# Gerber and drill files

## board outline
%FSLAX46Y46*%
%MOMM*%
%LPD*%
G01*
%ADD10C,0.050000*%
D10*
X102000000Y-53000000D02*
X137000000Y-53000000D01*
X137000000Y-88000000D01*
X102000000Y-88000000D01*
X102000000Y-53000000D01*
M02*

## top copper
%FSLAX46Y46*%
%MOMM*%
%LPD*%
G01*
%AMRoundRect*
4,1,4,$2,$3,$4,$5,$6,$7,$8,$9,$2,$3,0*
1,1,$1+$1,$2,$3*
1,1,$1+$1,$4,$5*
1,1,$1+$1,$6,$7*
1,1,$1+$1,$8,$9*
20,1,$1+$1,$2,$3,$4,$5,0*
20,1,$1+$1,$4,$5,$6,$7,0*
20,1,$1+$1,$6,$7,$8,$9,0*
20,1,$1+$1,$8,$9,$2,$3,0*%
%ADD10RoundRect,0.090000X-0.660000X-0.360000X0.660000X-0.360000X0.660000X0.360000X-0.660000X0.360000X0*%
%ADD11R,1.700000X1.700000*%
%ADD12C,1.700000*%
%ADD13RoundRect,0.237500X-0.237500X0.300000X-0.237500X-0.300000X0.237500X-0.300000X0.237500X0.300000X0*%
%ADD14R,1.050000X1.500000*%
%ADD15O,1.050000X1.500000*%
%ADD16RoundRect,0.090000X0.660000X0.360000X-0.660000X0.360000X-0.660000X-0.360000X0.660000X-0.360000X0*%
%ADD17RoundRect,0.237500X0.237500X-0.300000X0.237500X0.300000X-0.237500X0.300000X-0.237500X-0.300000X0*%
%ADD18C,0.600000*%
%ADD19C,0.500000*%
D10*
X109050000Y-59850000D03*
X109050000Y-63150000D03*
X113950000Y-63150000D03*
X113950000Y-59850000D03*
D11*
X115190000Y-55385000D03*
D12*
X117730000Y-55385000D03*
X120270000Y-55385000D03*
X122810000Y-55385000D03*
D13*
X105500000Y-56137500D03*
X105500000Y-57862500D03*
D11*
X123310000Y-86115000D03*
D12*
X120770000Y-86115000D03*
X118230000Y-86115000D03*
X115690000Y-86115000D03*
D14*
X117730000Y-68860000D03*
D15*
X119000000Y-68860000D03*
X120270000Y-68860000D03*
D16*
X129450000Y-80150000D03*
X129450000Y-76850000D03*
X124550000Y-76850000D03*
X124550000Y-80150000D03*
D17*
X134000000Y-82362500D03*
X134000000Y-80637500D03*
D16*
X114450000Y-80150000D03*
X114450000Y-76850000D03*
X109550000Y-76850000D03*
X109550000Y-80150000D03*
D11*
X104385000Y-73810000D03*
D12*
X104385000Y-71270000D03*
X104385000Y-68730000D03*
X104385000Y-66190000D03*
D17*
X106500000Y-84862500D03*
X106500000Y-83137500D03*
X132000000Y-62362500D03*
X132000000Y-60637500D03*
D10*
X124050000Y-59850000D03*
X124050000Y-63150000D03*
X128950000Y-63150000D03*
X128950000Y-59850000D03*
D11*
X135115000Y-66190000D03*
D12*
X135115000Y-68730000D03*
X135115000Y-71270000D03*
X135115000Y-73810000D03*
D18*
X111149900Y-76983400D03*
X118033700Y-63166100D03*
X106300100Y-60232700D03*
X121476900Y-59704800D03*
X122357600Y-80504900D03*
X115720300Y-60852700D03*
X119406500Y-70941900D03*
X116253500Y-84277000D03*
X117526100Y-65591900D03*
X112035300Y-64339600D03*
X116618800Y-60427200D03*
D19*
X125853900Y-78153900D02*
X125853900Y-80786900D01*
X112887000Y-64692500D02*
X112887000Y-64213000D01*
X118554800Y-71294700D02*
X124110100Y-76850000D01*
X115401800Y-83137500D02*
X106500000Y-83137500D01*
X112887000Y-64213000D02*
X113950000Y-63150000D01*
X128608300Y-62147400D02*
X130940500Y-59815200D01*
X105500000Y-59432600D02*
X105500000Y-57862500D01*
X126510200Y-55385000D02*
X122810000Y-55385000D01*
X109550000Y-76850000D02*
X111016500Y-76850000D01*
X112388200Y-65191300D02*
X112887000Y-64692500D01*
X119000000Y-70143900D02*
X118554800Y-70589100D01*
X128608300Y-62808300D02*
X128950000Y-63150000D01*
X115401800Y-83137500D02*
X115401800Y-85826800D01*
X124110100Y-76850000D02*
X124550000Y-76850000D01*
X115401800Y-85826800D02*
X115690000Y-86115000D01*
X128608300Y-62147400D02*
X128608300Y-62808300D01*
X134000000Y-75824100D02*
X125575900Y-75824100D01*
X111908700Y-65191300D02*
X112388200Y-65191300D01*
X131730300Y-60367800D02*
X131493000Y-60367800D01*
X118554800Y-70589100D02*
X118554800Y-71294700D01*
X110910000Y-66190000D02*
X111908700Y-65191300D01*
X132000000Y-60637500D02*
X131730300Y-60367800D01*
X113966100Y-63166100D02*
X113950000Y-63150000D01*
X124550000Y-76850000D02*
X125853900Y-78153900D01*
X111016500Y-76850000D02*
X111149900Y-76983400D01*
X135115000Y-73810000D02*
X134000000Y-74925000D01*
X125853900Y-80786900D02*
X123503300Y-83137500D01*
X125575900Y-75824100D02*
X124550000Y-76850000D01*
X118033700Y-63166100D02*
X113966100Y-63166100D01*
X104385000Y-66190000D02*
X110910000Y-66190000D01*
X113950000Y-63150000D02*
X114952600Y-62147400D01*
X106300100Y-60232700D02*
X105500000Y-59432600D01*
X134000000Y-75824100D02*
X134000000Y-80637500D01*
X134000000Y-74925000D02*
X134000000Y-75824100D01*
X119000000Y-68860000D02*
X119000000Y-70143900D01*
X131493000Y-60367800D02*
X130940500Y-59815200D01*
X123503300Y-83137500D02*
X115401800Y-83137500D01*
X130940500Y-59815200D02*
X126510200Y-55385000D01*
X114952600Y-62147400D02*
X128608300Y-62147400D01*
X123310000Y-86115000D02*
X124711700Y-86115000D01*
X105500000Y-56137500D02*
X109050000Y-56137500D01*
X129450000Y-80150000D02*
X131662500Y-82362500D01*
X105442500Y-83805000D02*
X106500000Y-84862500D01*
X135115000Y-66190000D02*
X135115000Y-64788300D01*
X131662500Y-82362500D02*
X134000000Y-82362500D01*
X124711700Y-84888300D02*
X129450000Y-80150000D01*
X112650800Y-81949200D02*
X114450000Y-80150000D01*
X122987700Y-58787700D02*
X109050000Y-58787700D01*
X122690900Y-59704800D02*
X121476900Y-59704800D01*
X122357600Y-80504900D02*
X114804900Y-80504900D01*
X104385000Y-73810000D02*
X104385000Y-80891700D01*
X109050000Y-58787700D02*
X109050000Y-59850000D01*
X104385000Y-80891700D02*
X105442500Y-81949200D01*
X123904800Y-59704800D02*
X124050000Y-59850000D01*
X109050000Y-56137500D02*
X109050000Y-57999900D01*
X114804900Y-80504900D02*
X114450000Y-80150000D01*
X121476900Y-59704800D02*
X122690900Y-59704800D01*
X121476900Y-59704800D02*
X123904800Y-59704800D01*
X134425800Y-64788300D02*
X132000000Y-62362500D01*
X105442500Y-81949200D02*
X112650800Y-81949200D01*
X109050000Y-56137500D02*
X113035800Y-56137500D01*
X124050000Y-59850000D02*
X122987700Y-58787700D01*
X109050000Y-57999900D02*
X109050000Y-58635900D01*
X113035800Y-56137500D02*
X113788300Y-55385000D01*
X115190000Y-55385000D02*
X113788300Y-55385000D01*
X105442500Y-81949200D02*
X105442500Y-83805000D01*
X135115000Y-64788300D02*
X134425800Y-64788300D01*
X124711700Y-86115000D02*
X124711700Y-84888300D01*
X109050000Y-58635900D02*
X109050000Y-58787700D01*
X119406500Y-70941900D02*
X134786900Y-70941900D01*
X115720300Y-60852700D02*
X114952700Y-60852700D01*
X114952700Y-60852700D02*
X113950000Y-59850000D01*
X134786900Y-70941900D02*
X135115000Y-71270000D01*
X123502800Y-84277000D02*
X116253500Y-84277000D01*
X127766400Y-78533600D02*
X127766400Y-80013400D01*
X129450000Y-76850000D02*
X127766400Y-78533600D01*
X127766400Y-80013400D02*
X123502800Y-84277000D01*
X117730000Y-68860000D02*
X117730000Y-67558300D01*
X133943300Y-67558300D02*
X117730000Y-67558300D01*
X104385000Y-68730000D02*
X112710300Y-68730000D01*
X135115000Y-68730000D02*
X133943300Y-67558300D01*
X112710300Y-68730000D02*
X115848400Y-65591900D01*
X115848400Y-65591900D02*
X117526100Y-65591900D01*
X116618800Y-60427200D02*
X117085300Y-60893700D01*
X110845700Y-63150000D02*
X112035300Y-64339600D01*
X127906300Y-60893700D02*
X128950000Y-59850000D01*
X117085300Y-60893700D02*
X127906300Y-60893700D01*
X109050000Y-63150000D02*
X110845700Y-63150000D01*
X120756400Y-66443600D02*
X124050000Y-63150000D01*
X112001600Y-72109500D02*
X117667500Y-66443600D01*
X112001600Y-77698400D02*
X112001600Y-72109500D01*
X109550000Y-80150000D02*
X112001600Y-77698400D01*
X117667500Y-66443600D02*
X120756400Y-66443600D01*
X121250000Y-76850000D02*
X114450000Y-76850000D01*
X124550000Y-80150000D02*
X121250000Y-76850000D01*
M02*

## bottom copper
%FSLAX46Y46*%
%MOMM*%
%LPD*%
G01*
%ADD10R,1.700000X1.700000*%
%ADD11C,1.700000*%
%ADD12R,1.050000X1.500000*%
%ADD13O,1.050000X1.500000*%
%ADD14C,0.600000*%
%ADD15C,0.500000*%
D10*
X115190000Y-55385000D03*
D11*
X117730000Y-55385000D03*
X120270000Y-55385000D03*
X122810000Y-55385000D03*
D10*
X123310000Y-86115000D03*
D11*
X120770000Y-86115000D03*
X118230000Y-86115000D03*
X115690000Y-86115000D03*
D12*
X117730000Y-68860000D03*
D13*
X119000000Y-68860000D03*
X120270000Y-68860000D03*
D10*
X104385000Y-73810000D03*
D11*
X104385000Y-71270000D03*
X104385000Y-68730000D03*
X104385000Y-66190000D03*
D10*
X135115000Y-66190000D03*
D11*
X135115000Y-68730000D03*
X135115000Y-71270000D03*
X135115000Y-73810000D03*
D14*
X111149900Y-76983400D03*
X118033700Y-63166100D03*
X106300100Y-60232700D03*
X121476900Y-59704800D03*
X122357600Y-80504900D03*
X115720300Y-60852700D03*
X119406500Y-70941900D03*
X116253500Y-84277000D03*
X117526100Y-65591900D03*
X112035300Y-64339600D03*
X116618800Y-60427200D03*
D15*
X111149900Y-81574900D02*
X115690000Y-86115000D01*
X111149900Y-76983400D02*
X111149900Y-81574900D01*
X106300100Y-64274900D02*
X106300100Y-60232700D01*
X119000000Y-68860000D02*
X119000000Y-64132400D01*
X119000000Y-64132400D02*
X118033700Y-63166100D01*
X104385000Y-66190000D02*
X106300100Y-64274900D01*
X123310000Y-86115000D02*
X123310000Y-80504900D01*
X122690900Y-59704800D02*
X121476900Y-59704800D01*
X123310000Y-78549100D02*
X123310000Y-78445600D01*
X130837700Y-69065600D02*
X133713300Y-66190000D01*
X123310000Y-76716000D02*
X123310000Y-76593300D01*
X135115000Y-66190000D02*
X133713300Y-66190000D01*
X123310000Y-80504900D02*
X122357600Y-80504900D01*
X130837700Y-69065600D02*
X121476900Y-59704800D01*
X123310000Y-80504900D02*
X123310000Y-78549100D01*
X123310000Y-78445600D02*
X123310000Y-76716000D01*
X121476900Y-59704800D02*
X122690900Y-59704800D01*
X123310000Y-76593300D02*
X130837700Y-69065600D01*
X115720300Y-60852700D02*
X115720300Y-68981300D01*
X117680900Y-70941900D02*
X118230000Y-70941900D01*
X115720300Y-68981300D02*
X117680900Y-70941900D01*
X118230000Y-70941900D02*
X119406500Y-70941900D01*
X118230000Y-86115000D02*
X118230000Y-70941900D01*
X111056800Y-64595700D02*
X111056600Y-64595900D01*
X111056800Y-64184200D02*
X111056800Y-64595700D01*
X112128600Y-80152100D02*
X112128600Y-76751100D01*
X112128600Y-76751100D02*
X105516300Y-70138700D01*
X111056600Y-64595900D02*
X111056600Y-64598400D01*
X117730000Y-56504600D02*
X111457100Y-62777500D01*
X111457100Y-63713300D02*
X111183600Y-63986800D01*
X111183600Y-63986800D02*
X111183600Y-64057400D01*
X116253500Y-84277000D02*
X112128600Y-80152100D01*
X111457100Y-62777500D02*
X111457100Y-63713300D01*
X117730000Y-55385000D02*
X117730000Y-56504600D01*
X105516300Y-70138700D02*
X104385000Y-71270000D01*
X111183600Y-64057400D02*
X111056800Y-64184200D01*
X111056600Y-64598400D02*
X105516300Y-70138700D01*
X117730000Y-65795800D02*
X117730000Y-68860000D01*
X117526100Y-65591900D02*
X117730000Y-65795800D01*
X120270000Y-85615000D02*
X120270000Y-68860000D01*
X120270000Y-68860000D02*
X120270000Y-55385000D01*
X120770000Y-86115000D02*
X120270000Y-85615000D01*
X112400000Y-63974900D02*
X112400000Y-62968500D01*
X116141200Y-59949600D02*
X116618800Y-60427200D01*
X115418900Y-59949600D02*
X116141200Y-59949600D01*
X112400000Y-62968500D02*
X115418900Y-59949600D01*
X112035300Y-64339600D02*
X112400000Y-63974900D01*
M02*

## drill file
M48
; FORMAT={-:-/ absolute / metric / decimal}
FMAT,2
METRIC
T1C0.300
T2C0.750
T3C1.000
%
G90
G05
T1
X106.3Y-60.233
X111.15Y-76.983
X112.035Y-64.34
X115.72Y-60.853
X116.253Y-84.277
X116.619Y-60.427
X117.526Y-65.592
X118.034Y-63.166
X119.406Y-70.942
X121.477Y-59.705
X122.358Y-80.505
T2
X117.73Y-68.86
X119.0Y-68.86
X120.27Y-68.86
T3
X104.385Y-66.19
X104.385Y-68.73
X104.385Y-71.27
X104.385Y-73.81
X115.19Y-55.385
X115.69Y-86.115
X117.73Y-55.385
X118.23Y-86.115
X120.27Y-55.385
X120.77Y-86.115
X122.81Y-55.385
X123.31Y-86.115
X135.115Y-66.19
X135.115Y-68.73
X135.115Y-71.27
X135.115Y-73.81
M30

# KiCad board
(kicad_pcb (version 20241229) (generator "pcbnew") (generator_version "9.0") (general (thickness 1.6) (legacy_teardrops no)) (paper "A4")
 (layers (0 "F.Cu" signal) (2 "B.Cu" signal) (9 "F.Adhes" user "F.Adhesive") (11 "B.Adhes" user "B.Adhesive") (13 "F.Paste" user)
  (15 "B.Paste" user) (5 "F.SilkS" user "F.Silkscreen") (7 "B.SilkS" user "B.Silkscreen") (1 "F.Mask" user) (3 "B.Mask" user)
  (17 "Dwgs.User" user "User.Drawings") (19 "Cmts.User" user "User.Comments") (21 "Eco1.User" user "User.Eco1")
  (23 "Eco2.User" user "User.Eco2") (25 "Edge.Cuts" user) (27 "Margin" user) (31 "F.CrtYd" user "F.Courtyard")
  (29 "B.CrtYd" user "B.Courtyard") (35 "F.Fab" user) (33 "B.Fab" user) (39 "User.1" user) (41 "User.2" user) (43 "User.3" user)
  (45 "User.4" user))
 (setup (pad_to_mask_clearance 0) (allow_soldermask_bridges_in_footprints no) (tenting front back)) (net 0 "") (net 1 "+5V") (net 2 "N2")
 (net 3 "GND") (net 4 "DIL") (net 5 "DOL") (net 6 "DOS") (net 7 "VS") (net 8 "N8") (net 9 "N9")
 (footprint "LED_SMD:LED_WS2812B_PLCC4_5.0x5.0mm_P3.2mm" (layer "F.Cu") (at 111.5 61.5)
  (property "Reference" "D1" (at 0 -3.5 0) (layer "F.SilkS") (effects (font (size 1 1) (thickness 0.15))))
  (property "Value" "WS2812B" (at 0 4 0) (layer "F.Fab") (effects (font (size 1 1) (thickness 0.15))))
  (pad "1" smd roundrect (at -2.45 -1.65) (size 1.5 0.9) (layers "F.Cu" "F.Mask" "F.Paste") (roundrect_rratio 0.1) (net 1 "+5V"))
  (pad "2" smd roundrect (at -2.45 1.65) (size 1.5 0.9) (layers "F.Cu" "F.Mask" "F.Paste") (roundrect_rratio 0.1) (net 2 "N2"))
  (pad "3" smd roundrect (at 2.45 1.65) (size 1.5 0.9) (layers "F.Cu" "F.Mask" "F.Paste") (roundrect_rratio 0.1) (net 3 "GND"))
  (pad "4" smd roundrect (at 2.45 -1.65) (size 1.5 0.9) (layers "F.Cu" "F.Mask" "F.Paste") (roundrect_rratio 0.1) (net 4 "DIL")))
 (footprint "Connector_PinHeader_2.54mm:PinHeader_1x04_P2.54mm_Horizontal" (layer "F.Cu") (at 115.19 55.385 90)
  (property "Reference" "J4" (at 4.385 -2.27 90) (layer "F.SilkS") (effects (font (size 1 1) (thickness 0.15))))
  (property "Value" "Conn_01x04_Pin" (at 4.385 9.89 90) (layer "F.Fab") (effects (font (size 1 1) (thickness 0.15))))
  (pad "1" thru_hole rect (at 0 0 90) (size 1.7 1.7) (drill 1) (layers "*.Cu" "*.Mask") (remove_unused_layers no) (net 1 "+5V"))
  (pad "2" thru_hole circle (at 0 2.54 90) (size 1.7 1.7) (drill 1) (layers "*.Cu" "*.Mask") (remove_unused_layers no) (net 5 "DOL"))
  (pad "3" thru_hole circle (at 0 5.08 90) (size 1.7 1.7) (drill 1) (layers "*.Cu" "*.Mask") (remove_unused_layers no) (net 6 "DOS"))
  (pad "4" thru_hole circle (at 0 7.62 90) (size 1.7 1.7) (drill 1) (layers "*.Cu" "*.Mask") (remove_unused_layers no) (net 3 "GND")))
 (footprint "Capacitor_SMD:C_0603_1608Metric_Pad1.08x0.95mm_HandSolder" (layer "F.Cu") (at 105.5 57 -90)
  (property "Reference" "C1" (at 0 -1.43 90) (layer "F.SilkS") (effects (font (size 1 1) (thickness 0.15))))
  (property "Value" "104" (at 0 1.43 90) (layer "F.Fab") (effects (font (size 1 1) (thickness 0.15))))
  (pad "1" smd roundrect (at -0.8625 0 270) (size 1.075 0.95) (layers "F.Cu" "F.Mask" "F.Paste") (roundrect_rratio 0.25) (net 1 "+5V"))
  (pad "2" smd roundrect (at 0.8625 0 270) (size 1.075 0.95) (layers "F.Cu" "F.Mask" "F.Paste") (roundrect_rratio 0.25) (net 3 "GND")))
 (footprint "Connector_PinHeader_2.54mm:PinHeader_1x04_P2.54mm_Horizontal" (layer "F.Cu") (at 123.31 86.115 -90)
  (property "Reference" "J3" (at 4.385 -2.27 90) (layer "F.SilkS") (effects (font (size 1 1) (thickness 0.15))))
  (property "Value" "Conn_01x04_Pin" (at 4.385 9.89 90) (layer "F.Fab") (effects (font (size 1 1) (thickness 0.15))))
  (pad "1" thru_hole rect (at 0 0 270) (size 1.7 1.7) (drill 1) (layers "*.Cu" "*.Mask") (remove_unused_layers no) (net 1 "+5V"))
  (pad "2" thru_hole circle (at 0 2.54 270) (size 1.7 1.7) (drill 1) (layers "*.Cu" "*.Mask") (remove_unused_layers no) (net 6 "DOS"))
  (pad "3" thru_hole circle (at 0 5.08 270) (size 1.7 1.7) (drill 1) (layers "*.Cu" "*.Mask") (remove_unused_layers no) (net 4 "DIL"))
  (pad "4" thru_hole circle (at 0 7.62 270) (size 1.7 1.7) (drill 1) (layers "*.Cu" "*.Mask") (remove_unused_layers no) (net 3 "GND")))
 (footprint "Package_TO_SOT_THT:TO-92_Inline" (layer "F.Cu") (at 117.73 68.86)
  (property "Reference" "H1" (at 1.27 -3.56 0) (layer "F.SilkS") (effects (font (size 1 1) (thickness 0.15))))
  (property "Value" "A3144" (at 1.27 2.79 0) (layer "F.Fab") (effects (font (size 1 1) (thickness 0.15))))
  (pad "1" thru_hole rect (at 0 0) (size 1.05 1.5) (drill 0.75) (layers "*.Cu" "*.Mask") (remove_unused_layers no) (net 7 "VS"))
  (pad "2" thru_hole oval (at 1.27 0) (size 1.05 1.5) (drill 0.75) (layers "*.Cu" "*.Mask") (remove_unused_layers no) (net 3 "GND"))
  (pad "3" thru_hole oval (at 2.54 0) (size 1.05 1.5) (drill 0.75) (layers "*.Cu" "*.Mask") (remove_unused_layers no) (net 6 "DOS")))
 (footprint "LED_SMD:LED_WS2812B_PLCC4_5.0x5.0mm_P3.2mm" (layer "F.Cu") (at 127 78.5 180)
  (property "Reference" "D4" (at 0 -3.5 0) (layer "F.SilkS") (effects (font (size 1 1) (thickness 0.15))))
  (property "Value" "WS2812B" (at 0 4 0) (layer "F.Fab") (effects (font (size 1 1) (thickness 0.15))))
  (pad "1" smd roundrect (at -2.45 -1.65 180) (size 1.5 0.9) (layers "F.Cu" "F.Mask" "F.Paste") (roundrect_rratio 0.1) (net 1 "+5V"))
  (pad "2" smd roundrect (at -2.45 1.65 180) (size 1.5 0.9) (layers "F.Cu" "F.Mask" "F.Paste") (roundrect_rratio 0.1) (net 5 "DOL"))
  (pad "3" smd roundrect (at 2.45 1.65 180) (size 1.5 0.9) (layers "F.Cu" "F.Mask" "F.Paste") (roundrect_rratio 0.1) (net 3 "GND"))
  (pad "4" smd roundrect (at 2.45 -1.65 180) (size 1.5 0.9) (layers "F.Cu" "F.Mask" "F.Paste") (roundrect_rratio 0.1) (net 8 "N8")))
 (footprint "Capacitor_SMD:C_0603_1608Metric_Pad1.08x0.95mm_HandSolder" (layer "F.Cu") (at 134 81.5 90)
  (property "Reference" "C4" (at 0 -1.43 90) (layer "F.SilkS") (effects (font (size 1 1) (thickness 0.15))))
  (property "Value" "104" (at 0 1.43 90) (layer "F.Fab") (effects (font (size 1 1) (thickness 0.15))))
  (pad "1" smd roundrect (at -0.8625 0 90) (size 1.075 0.95) (layers "F.Cu" "F.Mask" "F.Paste") (roundrect_rratio 0.25) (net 1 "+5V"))
  (pad "2" smd roundrect (at 0.8625 0 90) (size 1.075 0.95) (layers "F.Cu" "F.Mask" "F.Paste") (roundrect_rratio 0.25) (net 3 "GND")))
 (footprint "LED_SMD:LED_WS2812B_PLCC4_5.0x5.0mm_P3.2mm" (layer "F.Cu") (at 112 78.5 180)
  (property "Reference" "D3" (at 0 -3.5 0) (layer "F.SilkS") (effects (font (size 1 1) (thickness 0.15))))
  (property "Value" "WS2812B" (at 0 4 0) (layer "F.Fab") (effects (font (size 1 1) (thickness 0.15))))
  (pad "1" smd roundrect (at -2.45 -1.65 180) (size 1.5 0.9) (layers "F.Cu" "F.Mask" "F.Paste") (roundrect_rratio 0.1) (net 1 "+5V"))
  (pad "2" smd roundrect (at -2.45 1.65 180) (size 1.5 0.9) (layers "F.Cu" "F.Mask" "F.Paste") (roundrect_rratio 0.1) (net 8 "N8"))
  (pad "3" smd roundrect (at 2.45 1.65 180) (size 1.5 0.9) (layers "F.Cu" "F.Mask" "F.Paste") (roundrect_rratio 0.1) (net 3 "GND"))
  (pad "4" smd roundrect (at 2.45 -1.65 180) (size 1.5 0.9) (layers "F.Cu" "F.Mask" "F.Paste") (roundrect_rratio 0.1) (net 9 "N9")))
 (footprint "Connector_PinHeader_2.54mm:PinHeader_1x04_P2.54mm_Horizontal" (layer "F.Cu") (at 104.385 73.81 180)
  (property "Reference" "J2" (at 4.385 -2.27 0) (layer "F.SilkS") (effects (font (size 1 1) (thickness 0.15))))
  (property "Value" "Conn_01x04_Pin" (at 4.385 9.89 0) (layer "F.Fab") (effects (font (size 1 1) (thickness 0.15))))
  (pad "1" thru_hole rect (at 0 0 180) (size 1.7 1.7) (drill 1) (layers "*.Cu" "*.Mask") (remove_unused_layers no) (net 1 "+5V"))
  (pad "2" thru_hole circle (at 0 2.54 180) (size 1.7 1.7) (drill 1) (layers "*.Cu" "*.Mask") (remove_unused_layers no) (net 5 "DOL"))
  (pad "3" thru_hole circle (at 0 5.08 180) (size 1.7 1.7) (drill 1) (layers "*.Cu" "*.Mask") (remove_unused_layers no) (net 7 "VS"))
  (pad "4" thru_hole circle (at 0 7.62 180) (size 1.7 1.7) (drill 1) (layers "*.Cu" "*.Mask") (remove_unused_layers no) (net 3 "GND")))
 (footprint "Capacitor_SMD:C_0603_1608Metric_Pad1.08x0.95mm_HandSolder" (layer "F.Cu") (at 106.5 84 90)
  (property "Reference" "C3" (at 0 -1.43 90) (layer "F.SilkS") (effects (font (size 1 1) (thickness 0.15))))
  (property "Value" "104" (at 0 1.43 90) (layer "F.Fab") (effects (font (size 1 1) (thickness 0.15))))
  (pad "1" smd roundrect (at -0.8625 0 90) (size 1.075 0.95) (layers "F.Cu" "F.Mask" "F.Paste") (roundrect_rratio 0.25) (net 1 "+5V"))
  (pad "2" smd roundrect (at 0.8625 0 90) (size 1.075 0.95) (layers "F.Cu" "F.Mask" "F.Paste") (roundrect_rratio 0.25) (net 3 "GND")))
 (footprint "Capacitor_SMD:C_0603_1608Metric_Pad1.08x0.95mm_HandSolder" (layer "F.Cu") (at 132 61.5 90)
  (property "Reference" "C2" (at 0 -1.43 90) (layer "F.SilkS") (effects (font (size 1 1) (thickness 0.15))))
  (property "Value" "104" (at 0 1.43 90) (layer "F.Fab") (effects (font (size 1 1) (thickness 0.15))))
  (pad "1" smd roundrect (at -0.8625 0 90) (size 1.075 0.95) (layers "F.Cu" "F.Mask" "F.Paste") (roundrect_rratio 0.25) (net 1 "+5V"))
  (pad "2" smd roundrect (at 0.8625 0 90) (size 1.075 0.95) (layers "F.Cu" "F.Mask" "F.Paste") (roundrect_rratio 0.25) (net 3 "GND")))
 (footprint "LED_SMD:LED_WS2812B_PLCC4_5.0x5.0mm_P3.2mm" (layer "F.Cu") (at 126.5 61.5)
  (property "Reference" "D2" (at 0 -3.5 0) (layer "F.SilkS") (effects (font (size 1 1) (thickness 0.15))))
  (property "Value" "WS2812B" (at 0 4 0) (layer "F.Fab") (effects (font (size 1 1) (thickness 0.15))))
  (pad "1" smd roundrect (at -2.45 -1.65) (size 1.5 0.9) (layers "F.Cu" "F.Mask" "F.Paste") (roundrect_rratio 0.1) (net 1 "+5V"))
  (pad "2" smd roundrect (at -2.45 1.65) (size 1.5 0.9) (layers "F.Cu" "F.Mask" "F.Paste") (roundrect_rratio 0.1) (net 9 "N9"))
  (pad "3" smd roundrect (at 2.45 1.65) (size 1.5 0.9) (layers "F.Cu" "F.Mask" "F.Paste") (roundrect_rratio 0.1) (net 3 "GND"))
  (pad "4" smd roundrect (at 2.45 -1.65) (size 1.5 0.9) (layers "F.Cu" "F.Mask" "F.Paste") (roundrect_rratio 0.1) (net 2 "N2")))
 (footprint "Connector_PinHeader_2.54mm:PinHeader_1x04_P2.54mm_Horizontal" (layer "F.Cu") (at 135.115 66.19)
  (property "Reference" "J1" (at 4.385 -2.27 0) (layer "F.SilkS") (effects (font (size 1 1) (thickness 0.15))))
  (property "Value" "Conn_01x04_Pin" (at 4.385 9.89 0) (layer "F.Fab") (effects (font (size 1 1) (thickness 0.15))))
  (pad "1" thru_hole rect (at 0 0) (size 1.7 1.7) (drill 1) (layers "*.Cu" "*.Mask") (remove_unused_layers no) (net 1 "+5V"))
  (pad "2" thru_hole circle (at 0 2.54) (size 1.7 1.7) (drill 1) (layers "*.Cu" "*.Mask") (remove_unused_layers no) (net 7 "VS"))
  (pad "3" thru_hole circle (at 0 5.08) (size 1.7 1.7) (drill 1) (layers "*.Cu" "*.Mask") (remove_unused_layers no) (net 4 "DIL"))
  (pad "4" thru_hole circle (at 0 7.62) (size 1.7 1.7) (drill 1) (layers "*.Cu" "*.Mask") (remove_unused_layers no) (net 3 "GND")))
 (gr_rect (start 102 53) (end 137 88) (stroke (width 0.05) (type default)) (fill no) (layer "Edge.Cuts"))
 (segment (start 125.8539 78.1539) (end 125.8539 80.7869) (width 0.5) (layer "F.Cu") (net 3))
 (segment (start 112.887 64.6925) (end 112.887 64.213) (width 0.5) (layer "F.Cu") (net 3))
 (segment (start 118.5548 71.2947) (end 124.1101 76.85) (width 0.5) (layer "F.Cu") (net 3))
 (segment (start 115.4018 83.1375) (end 106.5 83.1375) (width 0.5) (layer "F.Cu") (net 3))
 (segment (start 112.887 64.213) (end 113.95 63.15) (width 0.5) (layer "F.Cu") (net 3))
 (segment (start 128.6083 62.1474) (end 130.9405 59.8152) (width 0.5) (layer "F.Cu") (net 3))
 (segment (start 105.5 59.4326) (end 105.5 57.8625) (width 0.5) (layer "F.Cu") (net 3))
 (segment (start 126.5102 55.385) (end 122.81 55.385) (width 0.5) (layer "F.Cu") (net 3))
 (segment (start 109.55 76.85) (end 111.0165 76.85) (width 0.5) (layer "F.Cu") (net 3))
 (segment (start 112.3882 65.1913) (end 112.887 64.6925) (width 0.5) (layer "F.Cu") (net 3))
 (segment (start 119 70.1439) (end 118.5548 70.5891) (width 0.5) (layer "F.Cu") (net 3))
 (segment (start 128.6083 62.8083) (end 128.95 63.15) (width 0.5) (layer "F.Cu") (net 3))
 (segment (start 115.4018 83.1375) (end 115.4018 85.8268) (width 0.5) (layer "F.Cu") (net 3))
 (segment (start 124.1101 76.85) (end 124.55 76.85) (width 0.5) (layer "F.Cu") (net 3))
 (segment (start 115.4018 85.8268) (end 115.69 86.115) (width 0.5) (layer "F.Cu") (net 3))
 (segment (start 128.6083 62.1474) (end 128.6083 62.8083) (width 0.5) (layer "F.Cu") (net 3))
 (segment (start 134 75.8241) (end 125.5759 75.8241) (width 0.5) (layer "F.Cu") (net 3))
 (segment (start 111.9087 65.1913) (end 112.3882 65.1913) (width 0.5) (layer "F.Cu") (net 3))
 (segment (start 131.7303 60.3678) (end 131.493 60.3678) (width 0.5) (layer "F.Cu") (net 3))
 (segment (start 118.5548 70.5891) (end 118.5548 71.2947) (width 0.5) (layer "F.Cu") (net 3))
 (segment (start 110.91 66.19) (end 111.9087 65.1913) (width 0.5) (layer "F.Cu") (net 3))
 (segment (start 132 60.6375) (end 131.7303 60.3678) (width 0.5) (layer "F.Cu") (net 3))
 (segment (start 113.9661 63.1661) (end 113.95 63.15) (width 0.5) (layer "F.Cu") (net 3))
 (segment (start 124.55 76.85) (end 125.8539 78.1539) (width 0.5) (layer "F.Cu") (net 3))
 (segment (start 111.0165 76.85) (end 111.1499 76.9834) (width 0.5) (layer "F.Cu") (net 3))
 (segment (start 135.115 73.81) (end 134 74.925) (width 0.5) (layer "F.Cu") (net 3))
 (segment (start 125.8539 80.7869) (end 123.5033 83.1375) (width 0.5) (layer "F.Cu") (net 3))
 (segment (start 125.5759 75.8241) (end 124.55 76.85) (width 0.5) (layer "F.Cu") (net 3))
 (segment (start 118.0337 63.1661) (end 113.9661 63.1661) (width 0.5) (layer "F.Cu") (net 3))
 (segment (start 104.385 66.19) (end 110.91 66.19) (width 0.5) (layer "F.Cu") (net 3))
 (segment (start 113.95 63.15) (end 114.9526 62.1474) (width 0.5) (layer "F.Cu") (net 3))
 (segment (start 106.3001 60.2327) (end 105.5 59.4326) (width 0.5) (layer "F.Cu") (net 3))
 (segment (start 134 75.8241) (end 134 80.6375) (width 0.5) (layer "F.Cu") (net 3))
 (segment (start 134 74.925) (end 134 75.8241) (width 0.5) (layer "F.Cu") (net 3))
 (segment (start 119 68.86) (end 119 70.1439) (width 0.5) (layer "F.Cu") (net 3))
 (segment (start 131.493 60.3678) (end 130.9405 59.8152) (width 0.5) (layer "F.Cu") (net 3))
 (segment (start 123.5033 83.1375) (end 115.4018 83.1375) (width 0.5) (layer "F.Cu") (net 3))
 (segment (start 130.9405 59.8152) (end 126.5102 55.385) (width 0.5) (layer "F.Cu") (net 3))
 (segment (start 114.9526 62.1474) (end 128.6083 62.1474) (width 0.5) (layer "F.Cu") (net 3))
 (via (at 111.1499 76.9834) (size 0.6) (drill 0.3) (layers "F.Cu" "B.Cu") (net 3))
 (via (at 118.0337 63.1661) (size 0.6) (drill 0.3) (layers "F.Cu" "B.Cu") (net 3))
 (via (at 106.3001 60.2327) (size 0.6) (drill 0.3) (layers "F.Cu" "B.Cu") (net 3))
 (segment (start 111.1499 81.5749) (end 115.69 86.115) (width 0.5) (layer "B.Cu") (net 3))
 (segment (start 111.1499 76.9834) (end 111.1499 81.5749) (width 0.5) (layer "B.Cu") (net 3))
 (segment (start 106.3001 64.2749) (end 106.3001 60.2327) (width 0.5) (layer "B.Cu") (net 3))
 (segment (start 119 68.86) (end 119 64.1324) (width 0.5) (layer "B.Cu") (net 3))
 (segment (start 119 64.1324) (end 118.0337 63.1661) (width 0.5) (layer "B.Cu") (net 3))
 (segment (start 104.385 66.19) (end 106.3001 64.2749) (width 0.5) (layer "B.Cu") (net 3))
 (segment (start 123.31 86.115) (end 124.7117 86.115) (width 0.5) (layer "F.Cu") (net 1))
 (segment (start 105.5 56.1375) (end 109.05 56.1375) (width 0.5) (layer "F.Cu") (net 1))
 (segment (start 129.45 80.15) (end 131.6625 82.3625) (width 0.5) (layer "F.Cu") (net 1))
 (segment (start 105.4425 83.805) (end 106.5 84.8625) (width 0.5) (layer "F.Cu") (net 1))
 (segment (start 135.115 66.19) (end 135.115 64.7883) (width 0.5) (layer "F.Cu") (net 1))
 (segment (start 131.6625 82.3625) (end 134 82.3625) (width 0.5) (layer "F.Cu") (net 1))
 (segment (start 124.7117 84.8883) (end 129.45 80.15) (width 0.5) (layer "F.Cu") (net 1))
 (segment (start 112.6508 81.9492) (end 114.45 80.15) (width 0.5) (layer "F.Cu") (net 1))
 (segment (start 122.9877 58.7877) (end 109.05 58.7877) (width 0.5) (layer "F.Cu") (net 1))
 (segment (start 122.6909 59.7048) (end 121.4769 59.7048) (width 0.5) (layer "F.Cu") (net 1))
 (segment (start 122.3576 80.5049) (end 114.8049 80.5049) (width 0.5) (layer "F.Cu") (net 1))
 (segment (start 104.385 73.81) (end 104.385 80.8917) (width 0.5) (layer "F.Cu") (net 1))
 (segment (start 109.05 58.7877) (end 109.05 59.85) (width 0.5) (layer "F.Cu") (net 1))
 (segment (start 104.385 80.8917) (end 105.4425 81.9492) (width 0.5) (layer "F.Cu") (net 1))
 (segment (start 123.9048 59.7048) (end 124.05 59.85) (width 0.5) (layer "F.Cu") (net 1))
 (segment (start 109.05 56.1375) (end 109.05 57.9999) (width 0.5) (layer "F.Cu") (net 1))
 (segment (start 114.8049 80.5049) (end 114.45 80.15) (width 0.5) (layer "F.Cu") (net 1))
 (segment (start 121.4769 59.7048) (end 122.6909 59.7048) (width 0.5) (layer "F.Cu") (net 1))
 (segment (start 121.4769 59.7048) (end 123.9048 59.7048) (width 0.5) (layer "F.Cu") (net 1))
 (segment (start 134.4258 64.7883) (end 132 62.3625) (width 0.5) (layer "F.Cu") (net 1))
 (segment (start 105.4425 81.9492) (end 112.6508 81.9492) (width 0.5) (layer "F.Cu") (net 1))
 (segment (start 109.05 56.1375) (end 113.0358 56.1375) (width 0.5) (layer "F.Cu") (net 1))
 (segment (start 124.05 59.85) (end 122.9877 58.7877) (width 0.5) (layer "F.Cu") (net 1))
 (segment (start 109.05 57.9999) (end 109.05 58.6359) (width 0.5) (layer "F.Cu") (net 1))
 (segment (start 113.0358 56.1375) (end 113.7883 55.385) (width 0.5) (layer "F.Cu") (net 1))
 (segment (start 115.19 55.385) (end 113.7883 55.385) (width 0.5) (layer "F.Cu") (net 1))
 (segment (start 105.4425 81.9492) (end 105.4425 83.805) (width 0.5) (layer "F.Cu") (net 1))
 (segment (start 135.115 64.7883) (end 134.4258 64.7883) (width 0.5) (layer "F.Cu") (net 1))
 (segment (start 124.7117 86.115) (end 124.7117 84.8883) (width 0.5) (layer "F.Cu") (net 1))
 (segment (start 109.05 58.6359) (end 109.05 58.7877) (width 0.5) (layer "F.Cu") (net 1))
 (via (at 121.4769 59.7048) (size 0.6) (drill 0.3) (layers "F.Cu" "B.Cu") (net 1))
 (via (at 122.3576 80.5049) (size 0.6) (drill 0.3) (layers "F.Cu" "B.Cu") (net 1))
 (segment (start 123.31 86.115) (end 123.31 80.5049) (width 0.5) (layer "B.Cu") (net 1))
 (segment (start 122.6909 59.7048) (end 121.4769 59.7048) (width 0.5) (layer "B.Cu") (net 1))
 (segment (start 123.31 78.5491) (end 123.31 78.4456) (width 0.5) (layer "B.Cu") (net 1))
 (segment (start 130.8377 69.0656) (end 133.7133 66.19) (width 0.5) (layer "B.Cu") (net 1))
 (segment (start 123.31 76.716) (end 123.31 76.5933) (width 0.5) (layer "B.Cu") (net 1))
 (segment (start 135.115 66.19) (end 133.7133 66.19) (width 0.5) (layer "B.Cu") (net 1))
 (segment (start 123.31 80.5049) (end 122.3576 80.5049) (width 0.5) (layer "B.Cu") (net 1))
 (segment (start 130.8377 69.0656) (end 121.4769 59.7048) (width 0.5) (layer "B.Cu") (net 1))
 (segment (start 123.31 80.5049) (end 123.31 78.5491) (width 0.5) (layer "B.Cu") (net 1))
 (segment (start 123.31 78.4456) (end 123.31 76.716) (width 0.5) (layer "B.Cu") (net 1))
 (segment (start 121.4769 59.7048) (end 122.6909 59.7048) (width 0.5) (layer "B.Cu") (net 1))
 (segment (start 123.31 76.5933) (end 130.8377 69.0656) (width 0.5) (layer "B.Cu") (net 1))
 (segment (start 119.4065 70.9419) (end 134.7869 70.9419) (width 0.5) (layer "F.Cu") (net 4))
 (segment (start 115.7203 60.8527) (end 114.9527 60.8527) (width 0.5) (layer "F.Cu") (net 4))
 (segment (start 114.9527 60.8527) (end 113.95 59.85) (width 0.5) (layer "F.Cu") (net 4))
 (segment (start 134.7869 70.9419) (end 135.115 71.27) (width 0.5) (layer "F.Cu") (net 4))
 (via (at 115.7203 60.8527) (size 0.6) (drill 0.3) (layers "F.Cu" "B.Cu") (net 4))
 (via (at 119.4065 70.9419) (size 0.6) (drill 0.3) (layers "F.Cu" "B.Cu") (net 4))
 (segment (start 115.7203 60.8527) (end 115.7203 68.9813) (width 0.5) (layer "B.Cu") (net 4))
 (segment (start 117.6809 70.9419) (end 118.23 70.9419) (width 0.5) (layer "B.Cu") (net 4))
 (segment (start 115.7203 68.9813) (end 117.6809 70.9419) (width 0.5) (layer "B.Cu") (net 4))
 (segment (start 118.23 70.9419) (end 119.4065 70.9419) (width 0.5) (layer "B.Cu") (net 4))
 (segment (start 118.23 86.115) (end 118.23 70.9419) (width 0.5) (layer "B.Cu") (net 4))
 (segment (start 123.5028 84.277) (end 116.2535 84.277) (width 0.5) (layer "F.Cu") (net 5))
 (segment (start 127.7664 78.5336) (end 127.7664 80.0134) (width 0.5) (layer "F.Cu") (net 5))
 (segment (start 129.45 76.85) (end 127.7664 78.5336) (width 0.5) (layer "F.Cu") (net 5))
 (segment (start 127.7664 80.0134) (end 123.5028 84.277) (width 0.5) (layer "F.Cu") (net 5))
 (via (at 116.2535 84.277) (size 0.6) (drill 0.3) (layers "F.Cu" "B.Cu") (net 5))
 (segment (start 111.0568 64.5957) (end 111.0566 64.5959) (width 0.5) (layer "B.Cu") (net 5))
 (segment (start 111.0568 64.1842) (end 111.0568 64.5957) (width 0.5) (layer "B.Cu") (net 5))
 (segment (start 112.1286 80.1521) (end 112.1286 76.7511) (width 0.5) (layer "B.Cu") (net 5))
 (segment (start 112.1286 76.7511) (end 105.5163 70.1387) (width 0.5) (layer "B.Cu") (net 5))
 (segment (start 111.0566 64.5959) (end 111.0566 64.5984) (width 0.5) (layer "B.Cu") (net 5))
 (segment (start 117.73 56.5046) (end 111.4571 62.7775) (width 0.5) (layer "B.Cu") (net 5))
 (segment (start 111.4571 63.7133) (end 111.1836 63.9868) (width 0.5) (layer "B.Cu") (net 5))
 (segment (start 111.1836 63.9868) (end 111.1836 64.0574) (width 0.5) (layer "B.Cu") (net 5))
 (segment (start 116.2535 84.277) (end 112.1286 80.1521) (width 0.5) (layer "B.Cu") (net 5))
 (segment (start 111.4571 62.7775) (end 111.4571 63.7133) (width 0.5) (layer "B.Cu") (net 5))
 (segment (start 117.73 55.385) (end 117.73 56.5046) (width 0.5) (layer "B.Cu") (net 5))
 (segment (start 105.5163 70.1387) (end 104.385 71.27) (width 0.5) (layer "B.Cu") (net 5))
 (segment (start 111.1836 64.0574) (end 111.0568 64.1842) (width 0.5) (layer "B.Cu") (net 5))
 (segment (start 111.0566 64.5984) (end 105.5163 70.1387) (width 0.5) (layer "B.Cu") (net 5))
 (segment (start 117.73 68.86) (end 117.73 67.5583) (width 0.5) (layer "F.Cu") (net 7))
 (segment (start 133.9433 67.5583) (end 117.73 67.5583) (width 0.5) (layer "F.Cu") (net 7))
 (segment (start 104.385 68.73) (end 112.7103 68.73) (width 0.5) (layer "F.Cu") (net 7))
 (segment (start 135.115 68.73) (end 133.9433 67.5583) (width 0.5) (layer "F.Cu") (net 7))
 (segment (start 112.7103 68.73) (end 115.8484 65.5919) (width 0.5) (layer "F.Cu") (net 7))
 (segment (start 115.8484 65.5919) (end 117.5261 65.5919) (width 0.5) (layer "F.Cu") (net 7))
 (via (at 117.5261 65.5919) (size 0.6) (drill 0.3) (layers "F.Cu" "B.Cu") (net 7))
 (segment (start 117.73 65.7958) (end 117.73 68.86) (width 0.5) (layer "B.Cu") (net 7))
 (segment (start 117.5261 65.5919) (end 117.73 65.7958) (width 0.5) (layer "B.Cu") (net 7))
 (segment (start 120.27 85.615) (end 120.27 68.86) (width 0.5) (layer "B.Cu") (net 6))
 (segment (start 120.27 68.86) (end 120.27 55.385) (width 0.5) (layer "B.Cu") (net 6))
 (segment (start 120.77 86.115) (end 120.27 85.615) (width 0.5) (layer "B.Cu") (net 6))
 (segment (start 116.6188 60.4272) (end 117.0853 60.8937) (width 0.5) (layer "F.Cu") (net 2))
 (segment (start 110.8457 63.15) (end 112.0353 64.3396) (width 0.5) (layer "F.Cu") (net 2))
 (segment (start 127.9063 60.8937) (end 128.95 59.85) (width 0.5) (layer "F.Cu") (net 2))
 (segment (start 117.0853 60.8937) (end 127.9063 60.8937) (width 0.5) (layer "F.Cu") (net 2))
 (segment (start 109.05 63.15) (end 110.8457 63.15) (width 0.5) (layer "F.Cu") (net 2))
 (via (at 112.0353 64.3396) (size 0.6) (drill 0.3) (layers "F.Cu" "B.Cu") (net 2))
 (via (at 116.6188 60.4272) (size 0.6) (drill 0.3) (layers "F.Cu" "B.Cu") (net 2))
 (segment (start 112.4 63.9749) (end 112.4 62.9685) (width 0.5) (layer "B.Cu") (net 2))
 (segment (start 116.1412 59.9496) (end 116.6188 60.4272) (width 0.5) (layer "B.Cu") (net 2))
 (segment (start 115.4189 59.9496) (end 116.1412 59.9496) (width 0.5) (layer "B.Cu") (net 2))
 (segment (start 112.4 62.9685) (end 115.4189 59.9496) (width 0.5) (layer "B.Cu") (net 2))
 (segment (start 112.0353 64.3396) (end 112.4 63.9749) (width 0.5) (layer "B.Cu") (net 2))
 (segment (start 120.7564 66.4436) (end 124.05 63.15) (width 0.5) (layer "F.Cu") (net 9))
 (segment (start 112.0016 72.1095) (end 117.6675 66.4436) (width 0.5) (layer "F.Cu") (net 9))
 (segment (start 112.0016 77.6984) (end 112.0016 72.1095) (width 0.5) (layer "F.Cu") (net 9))
 (segment (start 109.55 80.15) (end 112.0016 77.6984) (width 0.5) (layer "F.Cu") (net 9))
 (segment (start 117.6675 66.4436) (end 120.7564 66.4436) (width 0.5) (layer "F.Cu") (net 9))
 (segment (start 121.25 76.85) (end 114.45 76.85) (width 0.5) (layer "F.Cu") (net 8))
 (segment (start 124.55 80.15) (end 121.25 76.85) (width 0.5) (layer "F.Cu") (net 8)))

